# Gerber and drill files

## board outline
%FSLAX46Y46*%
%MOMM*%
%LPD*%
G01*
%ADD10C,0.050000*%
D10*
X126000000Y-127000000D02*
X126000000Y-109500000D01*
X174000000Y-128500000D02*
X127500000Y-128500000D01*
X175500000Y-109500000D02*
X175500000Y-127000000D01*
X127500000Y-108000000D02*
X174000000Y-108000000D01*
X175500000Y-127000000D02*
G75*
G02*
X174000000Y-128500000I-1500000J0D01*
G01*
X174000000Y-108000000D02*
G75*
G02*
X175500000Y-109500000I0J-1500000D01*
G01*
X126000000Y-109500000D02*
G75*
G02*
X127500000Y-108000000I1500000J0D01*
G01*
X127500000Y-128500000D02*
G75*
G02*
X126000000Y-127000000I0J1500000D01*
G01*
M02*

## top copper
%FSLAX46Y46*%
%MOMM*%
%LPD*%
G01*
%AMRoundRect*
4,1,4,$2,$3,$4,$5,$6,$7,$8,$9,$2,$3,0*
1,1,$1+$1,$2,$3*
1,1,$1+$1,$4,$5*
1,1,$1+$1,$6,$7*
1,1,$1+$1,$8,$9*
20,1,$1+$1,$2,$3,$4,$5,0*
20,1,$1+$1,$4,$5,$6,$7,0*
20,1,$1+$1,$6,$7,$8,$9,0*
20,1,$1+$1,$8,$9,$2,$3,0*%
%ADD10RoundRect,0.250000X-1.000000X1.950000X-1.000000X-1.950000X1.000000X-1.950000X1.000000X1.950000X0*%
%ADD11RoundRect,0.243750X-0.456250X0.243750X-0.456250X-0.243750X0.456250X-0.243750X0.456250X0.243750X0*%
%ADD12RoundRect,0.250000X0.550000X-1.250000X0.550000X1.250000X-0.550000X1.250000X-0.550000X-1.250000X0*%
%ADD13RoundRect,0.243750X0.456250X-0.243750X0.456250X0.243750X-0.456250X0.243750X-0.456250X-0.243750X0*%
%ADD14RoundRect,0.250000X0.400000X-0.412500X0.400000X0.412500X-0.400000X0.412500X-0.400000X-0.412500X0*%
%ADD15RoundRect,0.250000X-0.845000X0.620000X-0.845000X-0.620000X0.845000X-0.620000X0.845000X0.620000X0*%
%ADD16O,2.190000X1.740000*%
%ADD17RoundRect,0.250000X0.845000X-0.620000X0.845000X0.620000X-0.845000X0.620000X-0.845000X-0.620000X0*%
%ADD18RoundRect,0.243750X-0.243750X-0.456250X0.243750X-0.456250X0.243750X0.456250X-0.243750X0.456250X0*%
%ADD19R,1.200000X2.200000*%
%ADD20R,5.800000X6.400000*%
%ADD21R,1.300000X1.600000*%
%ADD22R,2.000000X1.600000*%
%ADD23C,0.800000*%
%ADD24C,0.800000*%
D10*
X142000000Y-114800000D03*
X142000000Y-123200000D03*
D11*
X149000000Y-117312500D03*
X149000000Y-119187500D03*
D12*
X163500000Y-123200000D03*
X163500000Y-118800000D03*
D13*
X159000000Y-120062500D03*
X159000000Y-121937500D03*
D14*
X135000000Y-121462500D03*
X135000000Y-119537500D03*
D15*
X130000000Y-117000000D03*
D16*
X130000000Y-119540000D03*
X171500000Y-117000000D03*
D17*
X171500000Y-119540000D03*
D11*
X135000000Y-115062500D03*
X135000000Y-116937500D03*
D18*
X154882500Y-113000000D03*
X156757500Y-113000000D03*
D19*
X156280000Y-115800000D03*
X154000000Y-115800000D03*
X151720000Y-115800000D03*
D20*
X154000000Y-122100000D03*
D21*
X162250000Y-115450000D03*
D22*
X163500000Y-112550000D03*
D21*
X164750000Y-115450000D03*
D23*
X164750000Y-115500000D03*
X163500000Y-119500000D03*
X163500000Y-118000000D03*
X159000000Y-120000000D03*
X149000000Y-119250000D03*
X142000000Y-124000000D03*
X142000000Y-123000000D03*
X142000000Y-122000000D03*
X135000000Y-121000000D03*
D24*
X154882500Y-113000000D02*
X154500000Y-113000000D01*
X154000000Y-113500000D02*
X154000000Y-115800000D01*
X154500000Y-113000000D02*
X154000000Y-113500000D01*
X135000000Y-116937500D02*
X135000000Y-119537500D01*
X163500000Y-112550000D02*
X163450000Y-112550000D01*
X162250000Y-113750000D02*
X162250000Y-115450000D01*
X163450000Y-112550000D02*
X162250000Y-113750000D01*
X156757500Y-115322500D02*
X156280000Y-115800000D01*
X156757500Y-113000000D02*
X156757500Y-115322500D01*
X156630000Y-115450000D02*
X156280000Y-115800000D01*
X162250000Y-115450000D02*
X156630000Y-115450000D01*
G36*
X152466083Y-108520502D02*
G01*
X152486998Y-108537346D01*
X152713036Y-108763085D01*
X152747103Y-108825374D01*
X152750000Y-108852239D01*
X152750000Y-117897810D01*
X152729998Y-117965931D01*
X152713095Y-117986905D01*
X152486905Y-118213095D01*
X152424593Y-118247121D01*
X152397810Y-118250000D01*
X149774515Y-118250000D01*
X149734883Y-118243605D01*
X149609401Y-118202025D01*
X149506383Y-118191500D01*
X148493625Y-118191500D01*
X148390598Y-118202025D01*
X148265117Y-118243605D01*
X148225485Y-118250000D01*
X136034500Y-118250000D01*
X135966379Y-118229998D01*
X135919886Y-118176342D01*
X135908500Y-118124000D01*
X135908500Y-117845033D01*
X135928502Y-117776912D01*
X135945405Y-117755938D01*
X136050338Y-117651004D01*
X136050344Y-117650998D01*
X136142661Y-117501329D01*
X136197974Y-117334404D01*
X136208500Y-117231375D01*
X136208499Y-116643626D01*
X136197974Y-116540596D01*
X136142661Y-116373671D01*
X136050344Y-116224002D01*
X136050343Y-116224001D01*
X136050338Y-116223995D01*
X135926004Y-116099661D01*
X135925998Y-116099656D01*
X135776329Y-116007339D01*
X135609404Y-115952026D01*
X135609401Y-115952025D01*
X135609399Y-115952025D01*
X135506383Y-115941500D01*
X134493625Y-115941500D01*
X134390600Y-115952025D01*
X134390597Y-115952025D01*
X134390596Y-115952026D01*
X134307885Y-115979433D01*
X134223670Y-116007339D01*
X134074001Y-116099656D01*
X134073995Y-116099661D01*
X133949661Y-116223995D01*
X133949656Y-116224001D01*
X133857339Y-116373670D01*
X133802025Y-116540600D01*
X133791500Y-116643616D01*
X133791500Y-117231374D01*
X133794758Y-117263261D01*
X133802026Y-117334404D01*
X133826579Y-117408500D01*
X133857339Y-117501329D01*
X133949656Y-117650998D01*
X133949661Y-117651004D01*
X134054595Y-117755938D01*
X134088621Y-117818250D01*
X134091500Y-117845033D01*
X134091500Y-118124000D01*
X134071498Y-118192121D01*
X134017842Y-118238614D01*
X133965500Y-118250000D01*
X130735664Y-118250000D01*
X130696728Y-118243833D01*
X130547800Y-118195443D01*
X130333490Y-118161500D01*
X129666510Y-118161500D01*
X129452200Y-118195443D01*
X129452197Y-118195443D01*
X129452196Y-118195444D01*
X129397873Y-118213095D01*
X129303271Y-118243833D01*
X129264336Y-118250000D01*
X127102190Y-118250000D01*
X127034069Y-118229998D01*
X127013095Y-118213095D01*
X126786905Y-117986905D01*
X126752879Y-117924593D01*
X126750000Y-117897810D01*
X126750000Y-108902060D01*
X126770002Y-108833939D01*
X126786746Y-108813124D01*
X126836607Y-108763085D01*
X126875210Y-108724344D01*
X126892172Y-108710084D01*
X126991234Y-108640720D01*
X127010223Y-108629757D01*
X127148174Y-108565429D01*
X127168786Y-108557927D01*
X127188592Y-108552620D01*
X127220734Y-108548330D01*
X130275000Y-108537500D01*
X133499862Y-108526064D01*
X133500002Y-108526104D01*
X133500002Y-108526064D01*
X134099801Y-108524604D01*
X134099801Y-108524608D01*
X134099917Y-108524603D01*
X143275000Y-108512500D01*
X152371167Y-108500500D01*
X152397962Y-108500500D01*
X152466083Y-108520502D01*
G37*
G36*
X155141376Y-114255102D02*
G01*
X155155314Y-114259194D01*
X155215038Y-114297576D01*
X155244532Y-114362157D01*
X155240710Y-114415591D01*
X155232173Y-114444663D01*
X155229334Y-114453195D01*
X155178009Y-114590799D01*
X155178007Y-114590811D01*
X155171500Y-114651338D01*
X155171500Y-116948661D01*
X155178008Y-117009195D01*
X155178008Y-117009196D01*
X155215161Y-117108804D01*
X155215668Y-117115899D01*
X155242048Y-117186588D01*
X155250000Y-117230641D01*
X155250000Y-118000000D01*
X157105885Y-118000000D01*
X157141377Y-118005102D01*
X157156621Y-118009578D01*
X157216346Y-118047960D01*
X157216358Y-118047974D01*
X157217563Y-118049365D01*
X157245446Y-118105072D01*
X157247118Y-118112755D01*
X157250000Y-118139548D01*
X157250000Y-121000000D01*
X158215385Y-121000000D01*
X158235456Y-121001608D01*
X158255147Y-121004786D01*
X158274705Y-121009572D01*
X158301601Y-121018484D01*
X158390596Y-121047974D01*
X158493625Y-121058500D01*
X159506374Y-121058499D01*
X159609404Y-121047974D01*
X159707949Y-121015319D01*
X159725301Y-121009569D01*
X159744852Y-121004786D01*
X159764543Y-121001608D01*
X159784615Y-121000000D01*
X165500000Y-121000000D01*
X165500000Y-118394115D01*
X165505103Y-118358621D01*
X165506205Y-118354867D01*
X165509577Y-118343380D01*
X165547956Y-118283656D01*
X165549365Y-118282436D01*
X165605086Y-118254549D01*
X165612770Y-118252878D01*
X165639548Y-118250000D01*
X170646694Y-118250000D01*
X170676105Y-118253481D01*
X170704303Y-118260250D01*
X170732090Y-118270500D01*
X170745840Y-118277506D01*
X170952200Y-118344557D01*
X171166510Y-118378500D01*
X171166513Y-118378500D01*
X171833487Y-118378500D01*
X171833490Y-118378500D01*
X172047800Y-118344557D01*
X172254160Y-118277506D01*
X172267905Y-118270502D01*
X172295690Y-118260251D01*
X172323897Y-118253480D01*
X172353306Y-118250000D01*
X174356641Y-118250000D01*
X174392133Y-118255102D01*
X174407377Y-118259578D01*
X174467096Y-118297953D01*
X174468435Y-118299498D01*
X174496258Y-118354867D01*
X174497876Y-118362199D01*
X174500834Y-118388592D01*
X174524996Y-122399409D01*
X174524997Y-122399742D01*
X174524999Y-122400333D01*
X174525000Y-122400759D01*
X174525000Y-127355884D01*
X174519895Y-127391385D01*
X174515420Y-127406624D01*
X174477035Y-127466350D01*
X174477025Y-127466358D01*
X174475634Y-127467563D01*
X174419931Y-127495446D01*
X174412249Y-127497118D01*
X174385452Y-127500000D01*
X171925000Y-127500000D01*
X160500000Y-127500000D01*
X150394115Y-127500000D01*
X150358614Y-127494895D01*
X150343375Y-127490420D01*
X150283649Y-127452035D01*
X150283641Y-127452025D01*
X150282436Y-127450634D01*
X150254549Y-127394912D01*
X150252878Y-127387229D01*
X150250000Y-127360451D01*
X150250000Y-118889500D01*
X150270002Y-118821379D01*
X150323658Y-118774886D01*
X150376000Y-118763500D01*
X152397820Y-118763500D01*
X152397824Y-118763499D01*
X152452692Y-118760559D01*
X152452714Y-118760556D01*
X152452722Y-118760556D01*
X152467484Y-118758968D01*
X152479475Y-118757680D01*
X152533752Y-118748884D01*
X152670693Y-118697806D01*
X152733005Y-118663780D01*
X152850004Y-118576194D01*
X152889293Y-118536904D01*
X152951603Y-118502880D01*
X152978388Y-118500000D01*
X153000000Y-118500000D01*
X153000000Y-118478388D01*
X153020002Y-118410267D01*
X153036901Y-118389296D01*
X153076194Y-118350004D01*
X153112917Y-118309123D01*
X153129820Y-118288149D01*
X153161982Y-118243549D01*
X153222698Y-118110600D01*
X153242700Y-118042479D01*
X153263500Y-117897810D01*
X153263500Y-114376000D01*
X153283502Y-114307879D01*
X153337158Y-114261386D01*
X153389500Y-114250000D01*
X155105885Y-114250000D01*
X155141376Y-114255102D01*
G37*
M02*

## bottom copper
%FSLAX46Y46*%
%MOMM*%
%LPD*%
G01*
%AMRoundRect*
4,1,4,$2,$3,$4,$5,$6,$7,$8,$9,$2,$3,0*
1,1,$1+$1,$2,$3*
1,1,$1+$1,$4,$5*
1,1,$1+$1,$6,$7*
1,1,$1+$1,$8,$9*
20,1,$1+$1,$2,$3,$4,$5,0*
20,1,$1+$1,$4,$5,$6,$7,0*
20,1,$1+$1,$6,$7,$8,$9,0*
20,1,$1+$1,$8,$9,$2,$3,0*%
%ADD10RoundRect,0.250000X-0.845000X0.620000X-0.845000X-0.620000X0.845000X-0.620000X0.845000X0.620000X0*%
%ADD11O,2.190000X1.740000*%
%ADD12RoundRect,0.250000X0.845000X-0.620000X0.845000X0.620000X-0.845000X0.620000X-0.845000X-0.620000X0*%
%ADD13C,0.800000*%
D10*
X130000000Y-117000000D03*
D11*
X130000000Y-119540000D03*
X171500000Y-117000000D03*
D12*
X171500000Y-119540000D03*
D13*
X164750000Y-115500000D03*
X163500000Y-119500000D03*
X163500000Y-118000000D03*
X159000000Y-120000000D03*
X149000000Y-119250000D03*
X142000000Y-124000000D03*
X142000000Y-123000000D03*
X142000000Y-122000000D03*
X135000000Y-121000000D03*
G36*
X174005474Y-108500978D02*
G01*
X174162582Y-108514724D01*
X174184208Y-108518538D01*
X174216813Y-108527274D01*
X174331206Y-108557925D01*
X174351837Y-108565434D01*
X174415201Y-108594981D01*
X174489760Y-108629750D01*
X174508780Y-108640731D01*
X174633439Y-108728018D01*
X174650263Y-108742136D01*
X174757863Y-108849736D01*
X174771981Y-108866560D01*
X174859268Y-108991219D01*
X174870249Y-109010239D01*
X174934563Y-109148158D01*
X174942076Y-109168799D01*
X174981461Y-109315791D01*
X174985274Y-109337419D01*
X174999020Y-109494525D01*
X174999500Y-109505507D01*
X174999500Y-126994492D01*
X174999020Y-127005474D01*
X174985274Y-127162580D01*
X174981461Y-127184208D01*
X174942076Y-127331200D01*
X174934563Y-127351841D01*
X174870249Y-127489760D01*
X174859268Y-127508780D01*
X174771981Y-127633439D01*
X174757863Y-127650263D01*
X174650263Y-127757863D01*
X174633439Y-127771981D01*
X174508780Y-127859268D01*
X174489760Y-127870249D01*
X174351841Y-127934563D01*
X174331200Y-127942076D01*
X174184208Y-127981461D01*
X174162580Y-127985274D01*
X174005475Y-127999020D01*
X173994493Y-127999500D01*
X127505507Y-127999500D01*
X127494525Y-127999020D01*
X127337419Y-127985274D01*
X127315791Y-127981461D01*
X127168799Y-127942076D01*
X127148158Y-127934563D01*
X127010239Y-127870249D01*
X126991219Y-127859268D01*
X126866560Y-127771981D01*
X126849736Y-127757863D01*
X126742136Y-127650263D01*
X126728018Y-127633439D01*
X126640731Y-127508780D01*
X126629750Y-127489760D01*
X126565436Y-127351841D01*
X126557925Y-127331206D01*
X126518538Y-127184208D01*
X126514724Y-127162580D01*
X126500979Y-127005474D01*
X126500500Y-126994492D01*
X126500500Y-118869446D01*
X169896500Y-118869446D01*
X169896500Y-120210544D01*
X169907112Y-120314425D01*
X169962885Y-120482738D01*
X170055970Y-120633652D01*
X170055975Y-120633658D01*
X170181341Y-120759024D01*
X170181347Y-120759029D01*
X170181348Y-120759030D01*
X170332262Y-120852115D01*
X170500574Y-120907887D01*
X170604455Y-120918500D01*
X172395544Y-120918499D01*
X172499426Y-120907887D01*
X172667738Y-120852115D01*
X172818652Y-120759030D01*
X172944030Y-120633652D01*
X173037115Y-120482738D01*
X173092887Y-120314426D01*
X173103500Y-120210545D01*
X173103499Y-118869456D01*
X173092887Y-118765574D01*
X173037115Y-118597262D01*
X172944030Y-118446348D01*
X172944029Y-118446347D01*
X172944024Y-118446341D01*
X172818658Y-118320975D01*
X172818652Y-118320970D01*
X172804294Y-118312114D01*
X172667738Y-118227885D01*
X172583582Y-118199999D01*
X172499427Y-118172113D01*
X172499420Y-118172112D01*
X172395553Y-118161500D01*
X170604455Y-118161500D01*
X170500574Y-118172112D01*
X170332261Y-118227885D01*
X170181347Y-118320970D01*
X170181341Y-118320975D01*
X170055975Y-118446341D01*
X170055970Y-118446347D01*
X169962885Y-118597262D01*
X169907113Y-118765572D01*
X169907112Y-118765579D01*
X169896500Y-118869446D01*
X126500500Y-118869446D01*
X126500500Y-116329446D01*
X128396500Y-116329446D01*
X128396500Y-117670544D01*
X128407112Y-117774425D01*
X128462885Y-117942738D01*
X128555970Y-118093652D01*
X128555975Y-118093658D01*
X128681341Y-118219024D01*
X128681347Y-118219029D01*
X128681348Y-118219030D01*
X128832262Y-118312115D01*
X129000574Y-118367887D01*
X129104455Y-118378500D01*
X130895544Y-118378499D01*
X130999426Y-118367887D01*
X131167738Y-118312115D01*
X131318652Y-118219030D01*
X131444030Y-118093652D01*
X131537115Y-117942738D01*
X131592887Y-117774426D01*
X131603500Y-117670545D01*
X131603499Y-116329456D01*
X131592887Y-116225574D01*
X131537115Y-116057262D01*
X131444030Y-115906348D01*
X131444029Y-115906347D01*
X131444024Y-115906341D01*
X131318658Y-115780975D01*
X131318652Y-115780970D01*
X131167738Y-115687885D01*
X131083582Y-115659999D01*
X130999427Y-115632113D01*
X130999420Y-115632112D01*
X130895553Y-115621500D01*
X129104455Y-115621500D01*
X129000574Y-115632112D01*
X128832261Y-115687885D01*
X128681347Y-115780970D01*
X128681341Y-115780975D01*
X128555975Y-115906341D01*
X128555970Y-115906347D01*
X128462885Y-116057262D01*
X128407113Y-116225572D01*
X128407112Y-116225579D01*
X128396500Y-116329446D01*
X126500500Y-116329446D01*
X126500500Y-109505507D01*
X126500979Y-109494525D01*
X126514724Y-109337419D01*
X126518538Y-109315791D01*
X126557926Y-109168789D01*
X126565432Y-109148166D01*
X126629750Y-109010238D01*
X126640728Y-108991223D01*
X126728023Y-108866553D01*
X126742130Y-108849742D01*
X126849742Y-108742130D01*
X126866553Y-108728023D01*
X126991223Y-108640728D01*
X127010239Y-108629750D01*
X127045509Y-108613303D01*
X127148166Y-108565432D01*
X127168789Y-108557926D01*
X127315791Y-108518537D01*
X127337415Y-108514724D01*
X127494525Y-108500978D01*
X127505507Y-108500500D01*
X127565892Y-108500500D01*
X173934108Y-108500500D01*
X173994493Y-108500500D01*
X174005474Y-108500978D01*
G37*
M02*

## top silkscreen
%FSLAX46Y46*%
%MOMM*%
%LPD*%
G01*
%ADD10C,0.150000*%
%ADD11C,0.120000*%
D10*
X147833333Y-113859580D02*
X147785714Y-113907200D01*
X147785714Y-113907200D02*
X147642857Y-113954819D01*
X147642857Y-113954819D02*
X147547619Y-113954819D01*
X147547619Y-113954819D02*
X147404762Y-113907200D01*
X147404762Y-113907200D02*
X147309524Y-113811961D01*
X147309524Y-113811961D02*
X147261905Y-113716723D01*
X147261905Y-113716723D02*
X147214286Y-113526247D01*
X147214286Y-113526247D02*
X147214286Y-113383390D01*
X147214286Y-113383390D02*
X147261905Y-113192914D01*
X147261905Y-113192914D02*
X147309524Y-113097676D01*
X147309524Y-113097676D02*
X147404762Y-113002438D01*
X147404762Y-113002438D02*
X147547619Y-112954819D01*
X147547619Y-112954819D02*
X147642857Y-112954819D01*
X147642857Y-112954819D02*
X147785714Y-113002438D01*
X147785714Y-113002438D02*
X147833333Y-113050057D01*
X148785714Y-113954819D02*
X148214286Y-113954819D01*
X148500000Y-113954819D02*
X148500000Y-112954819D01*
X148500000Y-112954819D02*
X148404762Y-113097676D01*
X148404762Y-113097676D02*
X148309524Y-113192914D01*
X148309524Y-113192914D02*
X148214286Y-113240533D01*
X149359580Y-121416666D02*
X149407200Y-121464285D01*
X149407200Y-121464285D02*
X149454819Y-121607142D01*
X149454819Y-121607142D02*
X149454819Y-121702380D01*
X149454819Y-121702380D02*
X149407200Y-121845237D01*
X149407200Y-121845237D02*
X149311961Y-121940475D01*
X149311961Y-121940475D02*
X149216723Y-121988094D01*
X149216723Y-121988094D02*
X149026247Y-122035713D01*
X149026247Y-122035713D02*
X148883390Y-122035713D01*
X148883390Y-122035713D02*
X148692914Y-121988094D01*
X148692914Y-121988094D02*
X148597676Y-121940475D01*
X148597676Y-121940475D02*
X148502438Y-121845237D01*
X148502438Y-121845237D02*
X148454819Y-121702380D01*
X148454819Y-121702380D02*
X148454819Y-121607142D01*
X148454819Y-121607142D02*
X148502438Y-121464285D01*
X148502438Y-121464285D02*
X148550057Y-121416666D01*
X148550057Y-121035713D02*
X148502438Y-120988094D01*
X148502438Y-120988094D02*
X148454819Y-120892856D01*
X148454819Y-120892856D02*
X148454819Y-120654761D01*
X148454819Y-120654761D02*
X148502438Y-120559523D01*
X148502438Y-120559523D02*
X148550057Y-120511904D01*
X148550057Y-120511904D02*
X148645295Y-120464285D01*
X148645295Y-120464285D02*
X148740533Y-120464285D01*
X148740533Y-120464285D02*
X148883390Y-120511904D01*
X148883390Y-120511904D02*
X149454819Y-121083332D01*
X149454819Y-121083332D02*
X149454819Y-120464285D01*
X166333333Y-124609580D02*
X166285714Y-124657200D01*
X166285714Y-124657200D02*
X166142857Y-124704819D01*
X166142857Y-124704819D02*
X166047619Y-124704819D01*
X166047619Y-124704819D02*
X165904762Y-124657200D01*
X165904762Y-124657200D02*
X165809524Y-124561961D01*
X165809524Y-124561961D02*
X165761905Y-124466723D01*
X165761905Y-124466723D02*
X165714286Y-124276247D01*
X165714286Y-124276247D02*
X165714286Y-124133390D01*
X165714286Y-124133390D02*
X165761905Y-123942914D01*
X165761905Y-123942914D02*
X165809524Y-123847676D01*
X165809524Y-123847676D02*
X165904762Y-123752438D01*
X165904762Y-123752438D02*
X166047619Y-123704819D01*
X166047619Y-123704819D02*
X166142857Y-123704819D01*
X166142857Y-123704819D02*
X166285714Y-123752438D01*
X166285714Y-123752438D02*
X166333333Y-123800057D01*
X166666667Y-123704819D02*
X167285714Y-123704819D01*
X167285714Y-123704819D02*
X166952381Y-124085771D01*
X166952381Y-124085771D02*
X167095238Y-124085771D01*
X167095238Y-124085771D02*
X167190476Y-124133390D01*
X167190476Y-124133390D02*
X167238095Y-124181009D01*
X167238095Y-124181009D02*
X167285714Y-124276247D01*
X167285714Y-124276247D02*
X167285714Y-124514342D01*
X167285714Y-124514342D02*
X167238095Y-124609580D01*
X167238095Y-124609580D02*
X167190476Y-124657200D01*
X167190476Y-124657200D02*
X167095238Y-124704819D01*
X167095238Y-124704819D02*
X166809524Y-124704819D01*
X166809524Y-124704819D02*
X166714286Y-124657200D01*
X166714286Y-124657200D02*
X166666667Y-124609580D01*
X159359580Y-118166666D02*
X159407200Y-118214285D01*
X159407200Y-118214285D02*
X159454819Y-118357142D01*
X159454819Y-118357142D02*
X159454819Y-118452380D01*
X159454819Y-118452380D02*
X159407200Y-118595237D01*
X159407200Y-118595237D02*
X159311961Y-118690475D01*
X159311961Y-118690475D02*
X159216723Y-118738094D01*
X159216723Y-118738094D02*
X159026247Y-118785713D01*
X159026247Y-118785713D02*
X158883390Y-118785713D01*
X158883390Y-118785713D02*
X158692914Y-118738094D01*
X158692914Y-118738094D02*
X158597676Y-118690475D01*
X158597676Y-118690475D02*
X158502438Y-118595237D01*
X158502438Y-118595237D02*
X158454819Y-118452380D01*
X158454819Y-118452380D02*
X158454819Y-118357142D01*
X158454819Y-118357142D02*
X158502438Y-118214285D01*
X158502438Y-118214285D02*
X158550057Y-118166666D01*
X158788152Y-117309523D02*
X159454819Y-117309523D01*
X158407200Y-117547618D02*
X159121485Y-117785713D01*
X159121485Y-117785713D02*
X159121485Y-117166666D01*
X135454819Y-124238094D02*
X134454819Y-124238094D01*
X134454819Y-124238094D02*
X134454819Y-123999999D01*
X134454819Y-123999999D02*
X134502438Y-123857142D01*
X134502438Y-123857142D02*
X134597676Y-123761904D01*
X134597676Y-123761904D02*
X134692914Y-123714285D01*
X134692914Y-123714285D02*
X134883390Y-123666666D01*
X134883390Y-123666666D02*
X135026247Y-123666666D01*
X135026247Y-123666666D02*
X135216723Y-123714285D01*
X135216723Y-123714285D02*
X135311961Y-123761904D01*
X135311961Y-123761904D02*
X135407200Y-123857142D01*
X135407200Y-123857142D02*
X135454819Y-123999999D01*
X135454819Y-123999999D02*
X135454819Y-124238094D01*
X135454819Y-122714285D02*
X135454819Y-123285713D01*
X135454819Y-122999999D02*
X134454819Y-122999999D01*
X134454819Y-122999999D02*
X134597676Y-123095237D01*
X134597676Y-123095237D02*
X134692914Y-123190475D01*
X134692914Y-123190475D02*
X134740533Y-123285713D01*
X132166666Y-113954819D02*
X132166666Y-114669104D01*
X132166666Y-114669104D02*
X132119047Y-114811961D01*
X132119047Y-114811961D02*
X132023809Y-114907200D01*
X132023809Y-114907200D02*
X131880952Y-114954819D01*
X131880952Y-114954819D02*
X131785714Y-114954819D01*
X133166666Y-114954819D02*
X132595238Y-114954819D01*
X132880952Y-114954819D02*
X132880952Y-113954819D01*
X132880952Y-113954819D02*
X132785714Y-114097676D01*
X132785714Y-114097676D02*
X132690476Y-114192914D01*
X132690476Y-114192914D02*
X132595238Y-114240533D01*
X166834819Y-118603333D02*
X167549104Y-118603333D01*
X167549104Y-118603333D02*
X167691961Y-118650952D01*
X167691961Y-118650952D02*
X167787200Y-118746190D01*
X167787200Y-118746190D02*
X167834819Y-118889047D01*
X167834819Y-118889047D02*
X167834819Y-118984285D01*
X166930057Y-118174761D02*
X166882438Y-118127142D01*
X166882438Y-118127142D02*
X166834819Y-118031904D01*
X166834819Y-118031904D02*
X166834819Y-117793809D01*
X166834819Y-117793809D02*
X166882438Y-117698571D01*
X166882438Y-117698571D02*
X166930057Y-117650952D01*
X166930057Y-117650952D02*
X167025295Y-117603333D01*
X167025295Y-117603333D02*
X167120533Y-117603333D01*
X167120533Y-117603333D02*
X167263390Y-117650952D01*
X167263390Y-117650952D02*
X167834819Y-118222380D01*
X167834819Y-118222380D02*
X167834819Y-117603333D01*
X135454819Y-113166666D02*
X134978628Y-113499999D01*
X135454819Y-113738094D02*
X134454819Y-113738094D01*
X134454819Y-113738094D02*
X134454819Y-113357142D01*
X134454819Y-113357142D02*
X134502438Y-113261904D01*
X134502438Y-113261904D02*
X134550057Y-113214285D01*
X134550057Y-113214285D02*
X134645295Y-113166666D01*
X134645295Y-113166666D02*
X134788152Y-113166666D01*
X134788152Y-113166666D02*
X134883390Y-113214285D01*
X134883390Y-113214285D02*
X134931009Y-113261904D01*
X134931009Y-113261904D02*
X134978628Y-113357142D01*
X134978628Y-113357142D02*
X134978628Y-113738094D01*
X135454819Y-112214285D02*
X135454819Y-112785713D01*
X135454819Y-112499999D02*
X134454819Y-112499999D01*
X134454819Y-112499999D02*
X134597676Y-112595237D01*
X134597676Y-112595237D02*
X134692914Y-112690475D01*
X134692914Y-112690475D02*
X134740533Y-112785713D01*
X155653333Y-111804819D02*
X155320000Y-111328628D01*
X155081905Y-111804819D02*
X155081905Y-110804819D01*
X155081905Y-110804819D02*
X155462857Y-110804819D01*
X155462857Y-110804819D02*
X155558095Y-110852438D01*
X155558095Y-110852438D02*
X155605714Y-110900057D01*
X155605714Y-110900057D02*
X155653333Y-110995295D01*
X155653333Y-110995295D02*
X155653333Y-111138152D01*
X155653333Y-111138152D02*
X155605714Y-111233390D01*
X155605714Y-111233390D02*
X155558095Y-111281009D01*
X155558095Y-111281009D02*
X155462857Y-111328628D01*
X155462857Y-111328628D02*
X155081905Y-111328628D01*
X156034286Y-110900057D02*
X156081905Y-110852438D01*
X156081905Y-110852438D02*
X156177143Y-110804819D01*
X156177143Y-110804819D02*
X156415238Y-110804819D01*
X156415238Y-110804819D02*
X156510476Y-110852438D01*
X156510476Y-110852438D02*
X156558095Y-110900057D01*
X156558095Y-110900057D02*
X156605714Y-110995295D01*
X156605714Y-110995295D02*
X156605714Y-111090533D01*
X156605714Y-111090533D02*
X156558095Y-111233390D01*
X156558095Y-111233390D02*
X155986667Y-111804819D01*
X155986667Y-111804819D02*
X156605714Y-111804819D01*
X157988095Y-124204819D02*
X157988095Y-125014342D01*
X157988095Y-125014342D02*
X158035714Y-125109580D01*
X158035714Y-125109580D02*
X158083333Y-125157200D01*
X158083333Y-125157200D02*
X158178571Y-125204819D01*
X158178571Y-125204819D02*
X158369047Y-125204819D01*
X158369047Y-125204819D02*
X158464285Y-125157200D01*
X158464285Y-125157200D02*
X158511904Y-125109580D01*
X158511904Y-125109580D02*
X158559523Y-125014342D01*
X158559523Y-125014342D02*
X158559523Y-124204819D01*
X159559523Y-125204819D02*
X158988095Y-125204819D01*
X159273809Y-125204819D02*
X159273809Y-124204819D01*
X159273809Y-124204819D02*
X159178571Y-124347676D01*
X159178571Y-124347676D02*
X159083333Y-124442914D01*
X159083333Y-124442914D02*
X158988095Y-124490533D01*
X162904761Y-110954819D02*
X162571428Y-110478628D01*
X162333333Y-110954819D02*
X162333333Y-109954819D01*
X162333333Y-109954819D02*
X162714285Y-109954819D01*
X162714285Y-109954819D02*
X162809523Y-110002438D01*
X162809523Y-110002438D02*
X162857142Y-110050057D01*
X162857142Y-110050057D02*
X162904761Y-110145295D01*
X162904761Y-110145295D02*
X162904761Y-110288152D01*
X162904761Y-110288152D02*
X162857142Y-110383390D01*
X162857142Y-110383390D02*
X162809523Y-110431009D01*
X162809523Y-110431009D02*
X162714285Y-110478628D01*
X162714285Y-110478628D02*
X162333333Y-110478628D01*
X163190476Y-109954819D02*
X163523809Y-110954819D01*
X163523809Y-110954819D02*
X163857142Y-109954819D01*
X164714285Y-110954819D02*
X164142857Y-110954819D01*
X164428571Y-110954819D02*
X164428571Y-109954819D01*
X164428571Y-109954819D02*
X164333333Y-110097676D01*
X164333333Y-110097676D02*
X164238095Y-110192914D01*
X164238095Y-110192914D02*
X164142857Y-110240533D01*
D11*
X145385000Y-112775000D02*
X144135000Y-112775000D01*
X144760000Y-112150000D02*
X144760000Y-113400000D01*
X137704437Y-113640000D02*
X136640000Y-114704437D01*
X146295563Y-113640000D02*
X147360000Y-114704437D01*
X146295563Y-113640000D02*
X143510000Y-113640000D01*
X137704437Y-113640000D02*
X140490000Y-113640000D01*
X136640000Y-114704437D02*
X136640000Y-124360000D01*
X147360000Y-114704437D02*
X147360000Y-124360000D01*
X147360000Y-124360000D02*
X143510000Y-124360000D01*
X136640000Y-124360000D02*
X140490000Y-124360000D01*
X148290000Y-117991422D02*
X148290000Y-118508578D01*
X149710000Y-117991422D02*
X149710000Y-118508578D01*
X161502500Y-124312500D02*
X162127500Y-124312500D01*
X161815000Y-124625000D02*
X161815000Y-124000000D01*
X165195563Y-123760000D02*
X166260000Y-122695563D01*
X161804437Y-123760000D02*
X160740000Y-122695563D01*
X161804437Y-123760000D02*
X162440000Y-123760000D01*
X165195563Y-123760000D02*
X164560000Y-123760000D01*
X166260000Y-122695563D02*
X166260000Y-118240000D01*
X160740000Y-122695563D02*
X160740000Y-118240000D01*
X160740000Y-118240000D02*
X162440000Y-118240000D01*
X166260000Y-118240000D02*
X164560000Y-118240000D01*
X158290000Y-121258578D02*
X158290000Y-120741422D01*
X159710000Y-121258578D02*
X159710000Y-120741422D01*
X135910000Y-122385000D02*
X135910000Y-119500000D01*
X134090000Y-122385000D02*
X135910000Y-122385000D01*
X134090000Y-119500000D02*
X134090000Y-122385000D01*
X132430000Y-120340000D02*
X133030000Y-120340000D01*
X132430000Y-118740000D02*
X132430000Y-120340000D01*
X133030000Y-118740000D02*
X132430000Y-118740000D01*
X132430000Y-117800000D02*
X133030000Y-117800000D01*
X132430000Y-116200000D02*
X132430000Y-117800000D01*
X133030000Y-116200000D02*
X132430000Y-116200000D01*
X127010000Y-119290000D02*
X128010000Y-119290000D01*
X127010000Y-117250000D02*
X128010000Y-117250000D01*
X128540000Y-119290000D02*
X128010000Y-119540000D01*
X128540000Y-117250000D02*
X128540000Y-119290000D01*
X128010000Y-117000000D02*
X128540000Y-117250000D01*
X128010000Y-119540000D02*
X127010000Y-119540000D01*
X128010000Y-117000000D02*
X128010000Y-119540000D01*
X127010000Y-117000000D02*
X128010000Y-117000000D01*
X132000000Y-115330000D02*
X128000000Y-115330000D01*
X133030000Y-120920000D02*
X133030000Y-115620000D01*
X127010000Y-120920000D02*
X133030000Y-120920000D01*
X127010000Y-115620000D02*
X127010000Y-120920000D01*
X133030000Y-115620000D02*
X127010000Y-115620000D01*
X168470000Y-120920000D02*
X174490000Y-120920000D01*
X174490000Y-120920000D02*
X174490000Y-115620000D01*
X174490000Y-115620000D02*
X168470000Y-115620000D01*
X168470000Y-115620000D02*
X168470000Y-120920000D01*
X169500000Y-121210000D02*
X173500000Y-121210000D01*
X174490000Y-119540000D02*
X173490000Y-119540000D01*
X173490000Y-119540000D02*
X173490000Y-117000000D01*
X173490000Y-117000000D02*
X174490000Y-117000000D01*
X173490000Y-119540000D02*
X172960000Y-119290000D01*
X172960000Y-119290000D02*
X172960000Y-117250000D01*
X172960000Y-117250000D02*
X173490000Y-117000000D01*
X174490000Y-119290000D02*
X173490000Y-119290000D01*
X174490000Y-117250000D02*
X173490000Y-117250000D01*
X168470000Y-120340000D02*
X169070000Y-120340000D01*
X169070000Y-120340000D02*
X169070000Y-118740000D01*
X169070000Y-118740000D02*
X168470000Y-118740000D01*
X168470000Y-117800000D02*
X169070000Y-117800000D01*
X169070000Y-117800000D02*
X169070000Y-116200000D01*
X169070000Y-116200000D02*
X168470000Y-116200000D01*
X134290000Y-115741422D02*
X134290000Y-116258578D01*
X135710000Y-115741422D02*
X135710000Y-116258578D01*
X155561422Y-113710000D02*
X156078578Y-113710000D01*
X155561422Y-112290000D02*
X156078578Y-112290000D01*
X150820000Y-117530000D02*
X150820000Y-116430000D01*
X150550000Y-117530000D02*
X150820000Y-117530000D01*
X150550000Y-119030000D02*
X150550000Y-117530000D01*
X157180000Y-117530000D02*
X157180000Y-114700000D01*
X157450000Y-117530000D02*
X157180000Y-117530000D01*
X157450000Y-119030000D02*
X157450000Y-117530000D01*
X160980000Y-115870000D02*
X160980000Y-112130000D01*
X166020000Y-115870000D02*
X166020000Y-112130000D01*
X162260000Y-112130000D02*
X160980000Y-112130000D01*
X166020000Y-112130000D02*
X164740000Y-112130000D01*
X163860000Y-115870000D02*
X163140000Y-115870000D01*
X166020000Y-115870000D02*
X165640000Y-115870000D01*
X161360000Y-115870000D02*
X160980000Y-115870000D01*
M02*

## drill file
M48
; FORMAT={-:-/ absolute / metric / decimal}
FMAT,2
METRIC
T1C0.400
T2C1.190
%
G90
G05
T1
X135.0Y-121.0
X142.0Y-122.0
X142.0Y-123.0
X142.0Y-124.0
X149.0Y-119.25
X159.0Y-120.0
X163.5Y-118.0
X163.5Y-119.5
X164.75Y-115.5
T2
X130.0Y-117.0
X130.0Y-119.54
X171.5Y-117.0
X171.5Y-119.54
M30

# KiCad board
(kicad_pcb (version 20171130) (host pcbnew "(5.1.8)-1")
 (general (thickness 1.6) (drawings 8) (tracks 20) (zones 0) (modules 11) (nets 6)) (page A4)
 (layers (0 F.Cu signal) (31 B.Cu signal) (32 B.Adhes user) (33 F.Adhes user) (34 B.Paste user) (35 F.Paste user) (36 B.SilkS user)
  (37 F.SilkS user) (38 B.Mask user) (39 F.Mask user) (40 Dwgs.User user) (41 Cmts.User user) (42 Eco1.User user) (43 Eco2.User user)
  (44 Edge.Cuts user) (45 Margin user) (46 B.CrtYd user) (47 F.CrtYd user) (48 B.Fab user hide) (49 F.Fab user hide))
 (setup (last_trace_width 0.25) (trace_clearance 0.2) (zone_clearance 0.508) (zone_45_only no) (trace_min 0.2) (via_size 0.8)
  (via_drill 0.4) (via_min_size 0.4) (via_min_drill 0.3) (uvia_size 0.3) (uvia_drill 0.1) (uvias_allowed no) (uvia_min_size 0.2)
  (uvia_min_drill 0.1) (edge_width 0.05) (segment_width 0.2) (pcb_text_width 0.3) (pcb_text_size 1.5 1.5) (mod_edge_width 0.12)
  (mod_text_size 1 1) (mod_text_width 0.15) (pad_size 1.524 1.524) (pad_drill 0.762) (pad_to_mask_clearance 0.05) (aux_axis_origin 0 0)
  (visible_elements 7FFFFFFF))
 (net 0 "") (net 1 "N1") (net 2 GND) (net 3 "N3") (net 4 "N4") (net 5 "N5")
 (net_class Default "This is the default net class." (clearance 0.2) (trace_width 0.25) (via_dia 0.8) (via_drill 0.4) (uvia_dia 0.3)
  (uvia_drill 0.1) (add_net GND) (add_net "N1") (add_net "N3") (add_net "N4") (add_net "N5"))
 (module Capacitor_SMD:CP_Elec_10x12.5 (layer F.Cu) (at 142 119 270)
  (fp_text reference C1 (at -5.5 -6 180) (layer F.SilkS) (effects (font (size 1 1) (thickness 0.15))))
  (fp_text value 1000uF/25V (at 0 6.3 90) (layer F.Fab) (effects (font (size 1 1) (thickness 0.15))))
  (fp_line (start -6.225 -3.385) (end -6.225 -2.135) (layer F.SilkS) (width 0.12))
  (fp_line (start -6.85 -2.76) (end -5.6 -2.76) (layer F.SilkS) (width 0.12))
  (fp_line (start -5.36 4.295563) (end -4.295563 5.36) (layer F.SilkS) (width 0.12))
  (fp_line (start -5.36 -4.295563) (end -4.295563 -5.36) (layer F.SilkS) (width 0.12))
  (fp_line (start -5.36 -4.295563) (end -5.36 -1.51) (layer F.SilkS) (width 0.12))
  (fp_line (start -5.36 4.295563) (end -5.36 1.51) (layer F.SilkS) (width 0.12))
  (fp_line (start -4.295563 5.36) (end 5.36 5.36) (layer F.SilkS) (width 0.12))
  (fp_line (start -4.295563 -5.36) (end 5.36 -5.36) (layer F.SilkS) (width 0.12))
  (fp_line (start 5.36 -5.36) (end 5.36 -1.51) (layer F.SilkS) (width 0.12))
  (fp_line (start 5.36 5.36) (end 5.36 1.51) (layer F.SilkS) (width 0.12))
  (pad 1 smd roundrect (at -4.2 0 270) (size 4.4 2.5) (layers F.Cu F.Paste F.Mask) (roundrect_rratio 0.1) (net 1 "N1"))
  (pad 2 smd roundrect (at 4.2 0 270) (size 4.4 2.5) (layers F.Cu F.Paste F.Mask) (roundrect_rratio 0.1) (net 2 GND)))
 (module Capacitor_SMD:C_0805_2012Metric (layer F.Cu) (at 149 118.25 270)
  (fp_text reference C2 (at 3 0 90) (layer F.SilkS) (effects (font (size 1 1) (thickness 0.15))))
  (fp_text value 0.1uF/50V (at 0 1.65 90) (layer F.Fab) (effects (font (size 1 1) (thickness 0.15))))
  (fp_line (start -0.258578 0.71) (end 0.258578 0.71) (layer F.SilkS) (width 0.12))
  (fp_line (start -0.258578 -0.71) (end 0.258578 -0.71) (layer F.SilkS) (width 0.12))
  (pad 1 smd roundrect (at -0.9375 0 270) (size 0.975 1.4) (layers F.Cu F.Paste F.Mask) (roundrect_rratio 0.25) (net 1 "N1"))
  (pad 2 smd roundrect (at 0.9375 0 270) (size 0.975 1.4) (layers F.Cu F.Paste F.Mask) (roundrect_rratio 0.25) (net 2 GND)))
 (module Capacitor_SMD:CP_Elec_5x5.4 (layer F.Cu) (at 163.5 121 90)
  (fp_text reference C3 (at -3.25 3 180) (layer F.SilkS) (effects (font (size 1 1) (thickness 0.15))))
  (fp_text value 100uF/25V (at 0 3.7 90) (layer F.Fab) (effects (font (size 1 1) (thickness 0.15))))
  (fp_line (start -3.3125 -1.9975) (end -3.3125 -1.3725) (layer F.SilkS) (width 0.12))
  (fp_line (start -3.625 -1.685) (end -3 -1.685) (layer F.SilkS) (width 0.12))
  (fp_line (start -2.76 1.695563) (end -1.695563 2.76) (layer F.SilkS) (width 0.12))
  (fp_line (start -2.76 -1.695563) (end -1.695563 -2.76) (layer F.SilkS) (width 0.12))
  (fp_line (start -2.76 -1.695563) (end -2.76 -1.06) (layer F.SilkS) (width 0.12))
  (fp_line (start -2.76 1.695563) (end -2.76 1.06) (layer F.SilkS) (width 0.12))
  (fp_line (start -1.695563 2.76) (end 2.76 2.76) (layer F.SilkS) (width 0.12))
  (fp_line (start -1.695563 -2.76) (end 2.76 -2.76) (layer F.SilkS) (width 0.12))
  (fp_line (start 2.76 -2.76) (end 2.76 -1.06) (layer F.SilkS) (width 0.12))
  (fp_line (start 2.76 2.76) (end 2.76 1.06) (layer F.SilkS) (width 0.12))
  (pad 1 smd roundrect (at -2.2 0 90) (size 3 1.6) (layers F.Cu F.Paste F.Mask) (roundrect_rratio 0.15625) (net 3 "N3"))
  (pad 2 smd roundrect (at 2.2 0 90) (size 3 1.6) (layers F.Cu F.Paste F.Mask) (roundrect_rratio 0.15625) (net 2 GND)))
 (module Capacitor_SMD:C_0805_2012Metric (layer F.Cu) (at 159 121 90)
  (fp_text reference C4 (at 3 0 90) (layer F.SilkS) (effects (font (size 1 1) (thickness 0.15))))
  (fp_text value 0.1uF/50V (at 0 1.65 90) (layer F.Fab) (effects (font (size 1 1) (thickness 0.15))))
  (fp_line (start -0.258578 -0.71) (end 0.258578 -0.71) (layer F.SilkS) (width 0.12))
  (fp_line (start -0.258578 0.71) (end 0.258578 0.71) (layer F.SilkS) (width 0.12))
  (pad 2 smd roundrect (at 0.9375 0 90) (size 0.975 1.4) (layers F.Cu F.Paste F.Mask) (roundrect_rratio 0.25) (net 2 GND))
  (pad 1 smd roundrect (at -0.9375 0 90) (size 0.975 1.4) (layers F.Cu F.Paste F.Mask) (roundrect_rratio 0.25) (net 3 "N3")))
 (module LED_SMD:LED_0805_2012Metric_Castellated (layer F.Cu) (at 135 120.5 90)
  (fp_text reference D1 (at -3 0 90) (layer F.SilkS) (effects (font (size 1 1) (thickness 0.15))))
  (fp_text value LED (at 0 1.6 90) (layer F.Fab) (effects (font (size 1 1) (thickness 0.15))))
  (fp_line (start -1.885 0.91) (end 1 0.91) (layer F.SilkS) (width 0.12))
  (fp_line (start -1.885 -0.91) (end -1.885 0.91) (layer F.SilkS) (width 0.12))
  (fp_line (start 1 -0.91) (end -1.885 -0.91) (layer F.SilkS) (width 0.12))
  (pad 1 smd roundrect (at -0.9625 0 90) (size 1.325 1.3) (layers F.Cu F.Paste F.Mask) (roundrect_rratio 0.192308) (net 2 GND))
  (pad 2 smd roundrect (at 0.9625 0 90) (size 1.325 1.3) (layers F.Cu F.Paste F.Mask) (roundrect_rratio 0.192308) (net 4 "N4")))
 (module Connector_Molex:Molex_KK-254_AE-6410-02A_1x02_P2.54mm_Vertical (layer F.Cu) (at 130 117 270)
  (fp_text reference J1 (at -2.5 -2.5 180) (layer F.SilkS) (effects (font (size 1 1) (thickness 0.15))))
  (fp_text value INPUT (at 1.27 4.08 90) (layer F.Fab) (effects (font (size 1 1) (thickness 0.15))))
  (fp_line (start 3.34 -2.43) (end 3.34 -3.03) (layer F.SilkS) (width 0.12))
  (fp_line (start 1.74 -2.43) (end 3.34 -2.43) (layer F.SilkS) (width 0.12))
  (fp_line (start 1.74 -3.03) (end 1.74 -2.43) (layer F.SilkS) (width 0.12))
  (fp_line (start 0.8 -2.43) (end 0.8 -3.03) (layer F.SilkS) (width 0.12))
  (fp_line (start -0.8 -2.43) (end 0.8 -2.43) (layer F.SilkS) (width 0.12))
  (fp_line (start -0.8 -3.03) (end -0.8 -2.43) (layer F.SilkS) (width 0.12))
  (fp_line (start 2.29 2.99) (end 2.29 1.99) (layer F.SilkS) (width 0.12))
  (fp_line (start 0.25 2.99) (end 0.25 1.99) (layer F.SilkS) (width 0.12))
  (fp_line (start 2.29 1.46) (end 2.54 1.99) (layer F.SilkS) (width 0.12))
  (fp_line (start 0.25 1.46) (end 2.29 1.46) (layer F.SilkS) (width 0.12))
  (fp_line (start 0 1.99) (end 0.25 1.46) (layer F.SilkS) (width 0.12))
  (fp_line (start 2.54 1.99) (end 2.54 2.99) (layer F.SilkS) (width 0.12))
  (fp_line (start 0 1.99) (end 2.54 1.99) (layer F.SilkS) (width 0.12))
  (fp_line (start 0 2.99) (end 0 1.99) (layer F.SilkS) (width 0.12))
  (fp_line (start -1.67 -2) (end -1.67 2) (layer F.SilkS) (width 0.12))
  (fp_line (start 3.92 -3.03) (end -1.38 -3.03) (layer F.SilkS) (width 0.12))
  (fp_line (start 3.92 2.99) (end 3.92 -3.03) (layer F.SilkS) (width 0.12))
  (fp_line (start -1.38 2.99) (end 3.92 2.99) (layer F.SilkS) (width 0.12))
  (fp_line (start -1.38 -3.03) (end -1.38 2.99) (layer F.SilkS) (width 0.12))
  (pad 1 thru_hole roundrect (at 0 0 270) (size 1.74 2.19) (drill 1.19) (layers *.Cu *.Mask) (roundrect_rratio 0.143678) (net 1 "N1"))
  (pad 2 thru_hole oval (at 2.54 0 270) (size 1.74 2.19) (drill 1.19) (layers *.Cu *.Mask) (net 2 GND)))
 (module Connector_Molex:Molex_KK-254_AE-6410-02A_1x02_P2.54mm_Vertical (layer F.Cu) (at 171.5 119.54 90)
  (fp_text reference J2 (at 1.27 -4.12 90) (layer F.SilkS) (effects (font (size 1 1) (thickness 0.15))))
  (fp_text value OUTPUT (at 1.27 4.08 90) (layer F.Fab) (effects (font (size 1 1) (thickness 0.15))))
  (fp_line (start -1.38 -3.03) (end -1.38 2.99) (layer F.SilkS) (width 0.12))
  (fp_line (start -1.38 2.99) (end 3.92 2.99) (layer F.SilkS) (width 0.12))
  (fp_line (start 3.92 2.99) (end 3.92 -3.03) (layer F.SilkS) (width 0.12))
  (fp_line (start 3.92 -3.03) (end -1.38 -3.03) (layer F.SilkS) (width 0.12))
  (fp_line (start -1.67 -2) (end -1.67 2) (layer F.SilkS) (width 0.12))
  (fp_line (start 0 2.99) (end 0 1.99) (layer F.SilkS) (width 0.12))
  (fp_line (start 0 1.99) (end 2.54 1.99) (layer F.SilkS) (width 0.12))
  (fp_line (start 2.54 1.99) (end 2.54 2.99) (layer F.SilkS) (width 0.12))
  (fp_line (start 0 1.99) (end 0.25 1.46) (layer F.SilkS) (width 0.12))
  (fp_line (start 0.25 1.46) (end 2.29 1.46) (layer F.SilkS) (width 0.12))
  (fp_line (start 2.29 1.46) (end 2.54 1.99) (layer F.SilkS) (width 0.12))
  (fp_line (start 0.25 2.99) (end 0.25 1.99) (layer F.SilkS) (width 0.12))
  (fp_line (start 2.29 2.99) (end 2.29 1.99) (layer F.SilkS) (width 0.12))
  (fp_line (start -0.8 -3.03) (end -0.8 -2.43) (layer F.SilkS) (width 0.12))
  (fp_line (start -0.8 -2.43) (end 0.8 -2.43) (layer F.SilkS) (width 0.12))
  (fp_line (start 0.8 -2.43) (end 0.8 -3.03) (layer F.SilkS) (width 0.12))
  (fp_line (start 1.74 -3.03) (end 1.74 -2.43) (layer F.SilkS) (width 0.12))
  (fp_line (start 1.74 -2.43) (end 3.34 -2.43) (layer F.SilkS) (width 0.12))
  (fp_line (start 3.34 -2.43) (end 3.34 -3.03) (layer F.SilkS) (width 0.12))
  (pad 2 thru_hole oval (at 2.54 0 90) (size 1.74 2.19) (drill 1.19) (layers *.Cu *.Mask) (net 2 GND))
  (pad 1 thru_hole roundrect (at 0 0 90) (size 1.74 2.19) (drill 1.19) (layers *.Cu *.Mask) (roundrect_rratio 0.143678) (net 3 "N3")))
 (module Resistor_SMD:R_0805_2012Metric (layer F.Cu) (at 135 116 270)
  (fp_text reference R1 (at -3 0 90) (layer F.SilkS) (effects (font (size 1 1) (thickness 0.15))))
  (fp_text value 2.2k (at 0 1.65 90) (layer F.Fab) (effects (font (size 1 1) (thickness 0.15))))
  (fp_line (start -0.258578 0.71) (end 0.258578 0.71) (layer F.SilkS) (width 0.12))
  (fp_line (start -0.258578 -0.71) (end 0.258578 -0.71) (layer F.SilkS) (width 0.12))
  (pad 1 smd roundrect (at -0.9375 0 270) (size 0.975 1.4) (layers F.Cu F.Paste F.Mask) (roundrect_rratio 0.25) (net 1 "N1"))
  (pad 2 smd roundrect (at 0.9375 0 270) (size 0.975 1.4) (layers F.Cu F.Paste F.Mask) (roundrect_rratio 0.25) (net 4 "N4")))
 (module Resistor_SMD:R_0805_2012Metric (layer F.Cu) (at 155.82 113)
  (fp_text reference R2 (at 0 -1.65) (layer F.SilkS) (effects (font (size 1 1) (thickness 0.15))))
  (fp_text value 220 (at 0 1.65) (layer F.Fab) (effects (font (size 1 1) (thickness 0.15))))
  (fp_line (start -0.258578 0.71) (end 0.258578 0.71) (layer F.SilkS) (width 0.12))
  (fp_line (start -0.258578 -0.71) (end 0.258578 -0.71) (layer F.SilkS) (width 0.12))
  (pad 1 smd roundrect (at -0.9375 0) (size 0.975 1.4) (layers F.Cu F.Paste F.Mask) (roundrect_rratio 0.25) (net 3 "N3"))
  (pad 2 smd roundrect (at 0.9375 0) (size 0.975 1.4) (layers F.Cu F.Paste F.Mask) (roundrect_rratio 0.25) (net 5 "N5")))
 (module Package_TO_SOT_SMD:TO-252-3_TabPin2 (layer F.Cu) (at 154 120 270)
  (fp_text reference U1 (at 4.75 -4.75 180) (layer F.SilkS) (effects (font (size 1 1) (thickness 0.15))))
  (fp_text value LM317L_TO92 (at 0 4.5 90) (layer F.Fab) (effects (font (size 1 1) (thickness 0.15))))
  (fp_line (start -2.47 3.18) (end -3.57 3.18) (layer F.SilkS) (width 0.12))
  (fp_line (start -2.47 3.45) (end -2.47 3.18) (layer F.SilkS) (width 0.12))
  (fp_line (start -0.97 3.45) (end -2.47 3.45) (layer F.SilkS) (width 0.12))
  (fp_line (start -2.47 -3.18) (end -5.3 -3.18) (layer F.SilkS) (width 0.12))
  (fp_line (start -2.47 -3.45) (end -2.47 -3.18) (layer F.SilkS) (width 0.12))
  (fp_line (start -0.97 -3.45) (end -2.47 -3.45) (layer F.SilkS) (width 0.12))
  (pad 1 smd rect (at -4.2 -2.28 270) (size 2.2 1.2) (layers F.Cu F.Paste F.Mask) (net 5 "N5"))
  (pad 2 smd rect (at -4.2 0 270) (size 2.2 1.2) (layers F.Cu F.Paste F.Mask) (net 3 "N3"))
  (pad 3 smd rect (at -4.2 2.28 270) (size 2.2 1.2) (layers F.Cu F.Paste F.Mask) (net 1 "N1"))
  (pad 2 smd rect (at 2.1 0 270) (size 6.4 5.8) (layers F.Cu F.Mask) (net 3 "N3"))
  (pad "" smd rect (at 3.775 1.525 270) (size 3.05 2.75) (layers F.Paste))
  (pad "" smd rect (at 0.425 -1.525 270) (size 3.05 2.75) (layers F.Paste))
  (pad "" smd rect (at 3.775 -1.525 270) (size 3.05 2.75) (layers F.Paste))
  (pad "" smd rect (at 0.425 1.525 270) (size 3.05 2.75) (layers F.Paste)))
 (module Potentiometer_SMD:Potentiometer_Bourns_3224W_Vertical (layer F.Cu) (at 163.5 114 180)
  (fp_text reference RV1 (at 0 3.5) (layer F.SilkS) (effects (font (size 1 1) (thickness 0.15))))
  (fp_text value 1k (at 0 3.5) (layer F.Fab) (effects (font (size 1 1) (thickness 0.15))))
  (fp_line (start 2.52 -1.87) (end 2.52 1.87) (layer F.SilkS) (width 0.12))
  (fp_line (start -2.52 -1.87) (end -2.52 1.87) (layer F.SilkS) (width 0.12))
  (fp_line (start 1.24 1.87) (end 2.52 1.87) (layer F.SilkS) (width 0.12))
  (fp_line (start -2.52 1.87) (end -1.24 1.87) (layer F.SilkS) (width 0.12))
  (fp_line (start -0.36 -1.87) (end 0.36 -1.87) (layer F.SilkS) (width 0.12))
  (fp_line (start -2.52 -1.87) (end -2.14 -1.87) (layer F.SilkS) (width 0.12))
  (fp_line (start 2.14 -1.87) (end 2.52 -1.87) (layer F.SilkS) (width 0.12))
  (pad 1 smd rect (at 1.25 -1.45 180) (size 1.3 1.6) (layers F.Cu F.Paste F.Mask) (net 5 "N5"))
  (pad 2 smd rect (at 0 1.45 180) (size 2 1.6) (layers F.Cu F.Paste F.Mask) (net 5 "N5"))
  (pad 3 smd rect (at -1.25 -1.45 180) (size 1.3 1.6) (layers F.Cu F.Paste F.Mask) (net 2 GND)))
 (gr_line (start 126 127) (end 126 109.5) (layer Edge.Cuts) (width 0.05))
 (gr_line (start 174 128.5) (end 127.5 128.5) (layer Edge.Cuts) (width 0.05))
 (gr_line (start 175.5 109.5) (end 175.5 127) (layer Edge.Cuts) (width 0.05))
 (gr_line (start 127.5 108) (end 174 108) (layer Edge.Cuts) (width 0.05))
 (gr_arc (start 174 127) (end 174 128.5) (angle -90) (layer Edge.Cuts) (width 0.05))
 (gr_arc (start 174 109.5) (end 175.5 109.5) (angle -90) (layer Edge.Cuts) (width 0.05))
 (gr_arc (start 127.5 109.5) (end 127.5 108) (angle -90) (layer Edge.Cuts) (width 0.05))
 (gr_arc (start 127.5 127) (end 126 127) (angle -90) (layer Edge.Cuts) (width 0.05))
 (via (at 164.75 115.5) (size 0.8) (drill 0.4) (layers F.Cu B.Cu) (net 2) (status 30))
 (via (at 163.5 119.5) (size 0.8) (drill 0.4) (layers F.Cu B.Cu) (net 2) (status 30))
 (via (at 163.5 118) (size 0.8) (drill 0.4) (layers F.Cu B.Cu) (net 2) (status 30))
 (via (at 159 120) (size 0.8) (drill 0.4) (layers F.Cu B.Cu) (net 2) (status 30))
 (via (at 149 119.25) (size 0.8) (drill 0.4) (layers F.Cu B.Cu) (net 2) (status 30))
 (via (at 142 124) (size 0.8) (drill 0.4) (layers F.Cu B.Cu) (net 2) (status 30))
 (via (at 142 123) (size 0.8) (drill 0.4) (layers F.Cu B.Cu) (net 2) (status 30))
 (via (at 142 122) (size 0.8) (drill 0.4) (layers F.Cu B.Cu) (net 2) (status 30))
 (via (at 135 121) (size 0.8) (drill 0.4) (layers F.Cu B.Cu) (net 2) (status 30))
 (segment (start 154.8825 113) (end 154.5 113) (width 0.8) (layer F.Cu) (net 3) (status 30))
 (segment (start 154 113.5) (end 154 115.8) (width 0.8) (layer F.Cu) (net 3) (status 20))
 (segment (start 154.5 113) (end 154 113.5) (width 0.8) (layer F.Cu) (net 3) (status 10))
 (segment (start 135 116.9375) (end 135 119.5375) (width 0.8) (layer F.Cu) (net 4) (status 30))
 (segment (start 163.5 112.55) (end 163.45 112.55) (width 0.8) (layer F.Cu) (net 5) (status 30))
 (segment (start 162.25 113.75) (end 162.25 115.45) (width 0.8) (layer F.Cu) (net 5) (status 20))
 (segment (start 163.45 112.55) (end 162.25 113.75) (width 0.8) (layer F.Cu) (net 5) (status 10))
 (segment (start 156.7575 115.3225) (end 156.28 115.8) (width 0.8) (layer F.Cu) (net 5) (status 30))
 (segment (start 156.7575 113) (end 156.7575 115.3225) (width 0.8) (layer F.Cu) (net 5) (status 30))
 (segment (start 156.63 115.45) (end 156.28 115.8) (width 0.8) (layer F.Cu) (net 5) (status 30))
 (segment (start 162.25 115.45) (end 156.63 115.45) (width 0.8) (layer F.Cu) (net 5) (status 30))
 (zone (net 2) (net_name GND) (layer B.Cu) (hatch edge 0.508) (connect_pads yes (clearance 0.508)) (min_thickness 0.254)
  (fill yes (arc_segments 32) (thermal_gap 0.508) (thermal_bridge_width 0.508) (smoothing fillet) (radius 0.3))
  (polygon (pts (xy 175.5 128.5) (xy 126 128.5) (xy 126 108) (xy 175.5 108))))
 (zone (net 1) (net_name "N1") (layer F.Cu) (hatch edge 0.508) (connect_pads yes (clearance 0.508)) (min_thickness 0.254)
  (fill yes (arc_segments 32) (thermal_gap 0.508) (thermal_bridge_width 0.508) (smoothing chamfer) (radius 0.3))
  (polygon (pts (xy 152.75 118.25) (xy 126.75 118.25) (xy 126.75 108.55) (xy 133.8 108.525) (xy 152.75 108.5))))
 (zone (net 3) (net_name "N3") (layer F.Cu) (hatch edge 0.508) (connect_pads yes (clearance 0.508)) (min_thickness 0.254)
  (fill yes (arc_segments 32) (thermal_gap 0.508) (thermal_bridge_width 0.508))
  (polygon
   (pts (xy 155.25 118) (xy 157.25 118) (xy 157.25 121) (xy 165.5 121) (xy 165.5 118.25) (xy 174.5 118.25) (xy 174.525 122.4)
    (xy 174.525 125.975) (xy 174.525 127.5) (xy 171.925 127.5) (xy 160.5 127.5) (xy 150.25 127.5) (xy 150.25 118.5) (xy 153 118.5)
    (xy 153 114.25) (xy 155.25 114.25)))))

